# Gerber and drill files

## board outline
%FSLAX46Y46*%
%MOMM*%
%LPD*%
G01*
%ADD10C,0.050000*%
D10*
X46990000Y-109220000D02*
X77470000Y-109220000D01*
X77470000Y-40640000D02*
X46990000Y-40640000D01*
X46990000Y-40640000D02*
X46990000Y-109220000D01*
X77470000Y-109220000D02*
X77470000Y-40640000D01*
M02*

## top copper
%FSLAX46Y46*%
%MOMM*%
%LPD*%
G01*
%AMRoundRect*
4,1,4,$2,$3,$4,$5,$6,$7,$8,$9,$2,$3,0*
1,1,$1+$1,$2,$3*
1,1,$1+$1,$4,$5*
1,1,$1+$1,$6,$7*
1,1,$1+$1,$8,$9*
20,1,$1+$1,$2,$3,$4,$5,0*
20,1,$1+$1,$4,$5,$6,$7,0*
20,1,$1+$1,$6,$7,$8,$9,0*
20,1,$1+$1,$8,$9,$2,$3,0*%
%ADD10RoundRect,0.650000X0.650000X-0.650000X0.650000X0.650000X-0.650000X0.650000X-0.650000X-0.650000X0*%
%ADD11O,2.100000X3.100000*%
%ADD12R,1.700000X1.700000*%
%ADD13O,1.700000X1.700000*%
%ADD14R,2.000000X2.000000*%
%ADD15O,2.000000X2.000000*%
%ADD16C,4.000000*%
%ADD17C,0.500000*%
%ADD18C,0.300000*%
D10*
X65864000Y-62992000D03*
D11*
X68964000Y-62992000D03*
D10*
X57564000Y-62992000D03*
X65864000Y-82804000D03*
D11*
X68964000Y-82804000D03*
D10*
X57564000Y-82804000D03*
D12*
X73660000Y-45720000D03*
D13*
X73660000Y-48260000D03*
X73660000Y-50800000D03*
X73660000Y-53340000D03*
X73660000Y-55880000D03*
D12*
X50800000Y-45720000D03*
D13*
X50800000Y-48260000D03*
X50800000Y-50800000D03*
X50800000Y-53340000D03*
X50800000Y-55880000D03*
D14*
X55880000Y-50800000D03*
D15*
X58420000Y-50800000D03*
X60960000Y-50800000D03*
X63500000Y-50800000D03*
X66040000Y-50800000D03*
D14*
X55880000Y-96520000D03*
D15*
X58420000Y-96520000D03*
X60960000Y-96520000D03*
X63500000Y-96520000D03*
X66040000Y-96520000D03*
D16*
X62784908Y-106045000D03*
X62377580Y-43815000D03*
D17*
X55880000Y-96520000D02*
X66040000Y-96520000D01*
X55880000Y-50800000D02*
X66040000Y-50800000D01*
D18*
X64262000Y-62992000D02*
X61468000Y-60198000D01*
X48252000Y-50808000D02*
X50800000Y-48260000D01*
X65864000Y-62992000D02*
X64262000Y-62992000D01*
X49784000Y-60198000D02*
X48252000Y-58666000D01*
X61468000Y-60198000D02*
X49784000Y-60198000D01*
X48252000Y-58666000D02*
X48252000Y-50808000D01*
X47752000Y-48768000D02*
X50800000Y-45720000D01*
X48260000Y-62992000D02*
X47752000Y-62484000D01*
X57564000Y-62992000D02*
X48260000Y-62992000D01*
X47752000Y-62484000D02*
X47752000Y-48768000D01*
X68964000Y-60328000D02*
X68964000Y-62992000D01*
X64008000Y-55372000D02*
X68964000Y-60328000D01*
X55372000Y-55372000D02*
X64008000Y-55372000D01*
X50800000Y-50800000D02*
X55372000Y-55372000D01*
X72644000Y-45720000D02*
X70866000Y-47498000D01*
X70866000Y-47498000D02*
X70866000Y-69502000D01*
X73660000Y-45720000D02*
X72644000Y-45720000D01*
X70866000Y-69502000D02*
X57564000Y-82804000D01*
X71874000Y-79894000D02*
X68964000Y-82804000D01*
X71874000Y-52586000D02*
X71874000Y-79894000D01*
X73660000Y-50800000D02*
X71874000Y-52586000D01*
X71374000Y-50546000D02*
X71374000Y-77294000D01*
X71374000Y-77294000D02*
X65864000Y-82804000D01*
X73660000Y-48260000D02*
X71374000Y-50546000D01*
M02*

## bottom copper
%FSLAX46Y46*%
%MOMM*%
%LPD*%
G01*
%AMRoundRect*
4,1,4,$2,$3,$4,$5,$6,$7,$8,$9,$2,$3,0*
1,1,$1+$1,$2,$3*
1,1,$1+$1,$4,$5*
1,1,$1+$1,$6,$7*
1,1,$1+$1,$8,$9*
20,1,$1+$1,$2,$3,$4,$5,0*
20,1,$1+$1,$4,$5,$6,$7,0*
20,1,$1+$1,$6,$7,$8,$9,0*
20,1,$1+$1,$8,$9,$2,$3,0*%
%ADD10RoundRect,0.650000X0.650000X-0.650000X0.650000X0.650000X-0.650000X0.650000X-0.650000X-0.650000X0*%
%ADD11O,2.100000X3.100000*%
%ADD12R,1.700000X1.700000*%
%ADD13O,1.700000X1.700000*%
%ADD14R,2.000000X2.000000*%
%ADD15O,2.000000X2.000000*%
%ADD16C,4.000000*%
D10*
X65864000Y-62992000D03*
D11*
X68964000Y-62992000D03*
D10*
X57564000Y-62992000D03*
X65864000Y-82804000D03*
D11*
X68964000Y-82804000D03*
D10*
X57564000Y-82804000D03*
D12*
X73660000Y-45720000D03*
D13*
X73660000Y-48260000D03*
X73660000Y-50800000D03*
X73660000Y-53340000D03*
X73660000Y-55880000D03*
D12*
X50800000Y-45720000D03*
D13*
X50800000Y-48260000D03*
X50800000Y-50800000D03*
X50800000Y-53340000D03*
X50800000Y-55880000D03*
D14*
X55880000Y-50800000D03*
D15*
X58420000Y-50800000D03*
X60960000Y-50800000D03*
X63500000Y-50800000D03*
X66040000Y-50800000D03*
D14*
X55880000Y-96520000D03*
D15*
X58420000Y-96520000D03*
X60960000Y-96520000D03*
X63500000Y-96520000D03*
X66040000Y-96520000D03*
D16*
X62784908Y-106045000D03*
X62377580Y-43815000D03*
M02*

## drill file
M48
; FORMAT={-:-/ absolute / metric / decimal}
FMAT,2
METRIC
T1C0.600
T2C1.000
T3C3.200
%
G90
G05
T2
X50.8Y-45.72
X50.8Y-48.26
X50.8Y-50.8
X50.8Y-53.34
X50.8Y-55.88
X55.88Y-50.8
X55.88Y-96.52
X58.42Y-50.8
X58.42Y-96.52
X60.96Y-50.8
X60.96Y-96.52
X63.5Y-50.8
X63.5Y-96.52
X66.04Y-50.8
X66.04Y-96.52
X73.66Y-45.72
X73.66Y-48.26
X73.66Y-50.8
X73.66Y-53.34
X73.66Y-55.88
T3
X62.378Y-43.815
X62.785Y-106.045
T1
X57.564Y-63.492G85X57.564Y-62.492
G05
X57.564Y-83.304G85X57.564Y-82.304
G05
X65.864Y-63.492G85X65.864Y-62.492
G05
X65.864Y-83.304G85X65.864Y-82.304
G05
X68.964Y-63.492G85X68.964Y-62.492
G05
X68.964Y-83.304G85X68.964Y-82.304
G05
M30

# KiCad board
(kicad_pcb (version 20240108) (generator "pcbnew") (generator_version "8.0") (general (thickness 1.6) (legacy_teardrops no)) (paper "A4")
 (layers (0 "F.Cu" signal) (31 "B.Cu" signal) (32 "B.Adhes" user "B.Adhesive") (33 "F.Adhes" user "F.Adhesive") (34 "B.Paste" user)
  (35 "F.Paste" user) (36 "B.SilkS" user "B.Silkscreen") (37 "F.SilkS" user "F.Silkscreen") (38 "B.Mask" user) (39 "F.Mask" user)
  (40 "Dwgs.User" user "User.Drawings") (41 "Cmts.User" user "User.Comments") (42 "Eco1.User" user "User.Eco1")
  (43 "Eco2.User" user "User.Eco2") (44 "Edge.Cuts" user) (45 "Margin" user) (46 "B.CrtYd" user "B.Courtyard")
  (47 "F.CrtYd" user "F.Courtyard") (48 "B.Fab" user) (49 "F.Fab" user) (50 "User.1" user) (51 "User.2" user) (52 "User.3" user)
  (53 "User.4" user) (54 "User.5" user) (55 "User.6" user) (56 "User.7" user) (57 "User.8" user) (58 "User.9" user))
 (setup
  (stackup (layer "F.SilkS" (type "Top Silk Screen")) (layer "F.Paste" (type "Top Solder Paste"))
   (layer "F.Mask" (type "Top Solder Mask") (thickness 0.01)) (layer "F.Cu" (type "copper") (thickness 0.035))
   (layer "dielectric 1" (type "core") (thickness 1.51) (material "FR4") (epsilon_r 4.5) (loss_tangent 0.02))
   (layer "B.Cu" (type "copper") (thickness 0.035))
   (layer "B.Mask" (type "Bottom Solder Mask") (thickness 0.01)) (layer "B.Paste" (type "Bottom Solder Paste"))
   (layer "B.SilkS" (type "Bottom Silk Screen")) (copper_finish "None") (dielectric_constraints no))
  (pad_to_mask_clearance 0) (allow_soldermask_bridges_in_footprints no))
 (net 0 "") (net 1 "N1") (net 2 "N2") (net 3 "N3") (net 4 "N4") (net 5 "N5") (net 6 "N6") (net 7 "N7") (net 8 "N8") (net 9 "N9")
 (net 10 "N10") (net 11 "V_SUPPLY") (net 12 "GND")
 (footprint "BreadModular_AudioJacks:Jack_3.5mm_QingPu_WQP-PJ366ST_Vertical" (layer "F.Cu") (at 62.484 62.992 90)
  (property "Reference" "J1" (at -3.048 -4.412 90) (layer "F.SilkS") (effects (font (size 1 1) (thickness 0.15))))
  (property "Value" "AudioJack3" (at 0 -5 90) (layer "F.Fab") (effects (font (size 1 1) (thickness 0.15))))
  (pad "R" thru_hole roundrect (at 0 3.38 90) (size 2.6 2.6) (drill oval 1.6 0.6) (layers "*.Cu" "*.Mask") (remove_unused_layers no)
   (roundrect_rratio 0.25) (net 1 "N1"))
  (pad "S" thru_hole oval (at 0 6.48 90) (size 3.1 2.1) (drill oval 1.6 0.6) (layers "*.Cu" "*.Mask") (remove_unused_layers no) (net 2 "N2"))
  (pad "T" thru_hole roundrect (at 0 -4.92 90) (size 2.6 2.6) (drill oval 1.6 0.6) (layers "*.Cu" "*.Mask") (remove_unused_layers no)
   (roundrect_rratio 0.25) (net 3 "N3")))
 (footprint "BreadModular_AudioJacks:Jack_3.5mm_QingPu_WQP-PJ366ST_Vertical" (layer "F.Cu") (at 62.484 82.804 90)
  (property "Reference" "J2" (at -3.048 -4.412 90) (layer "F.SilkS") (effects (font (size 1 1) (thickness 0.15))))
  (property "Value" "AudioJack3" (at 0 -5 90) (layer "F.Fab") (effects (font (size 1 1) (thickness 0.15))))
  (pad "R" thru_hole roundrect (at 0 3.38 90) (size 2.6 2.6) (drill oval 1.6 0.6) (layers "*.Cu" "*.Mask") (remove_unused_layers no)
   (roundrect_rratio 0.25) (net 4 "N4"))
  (pad "S" thru_hole oval (at 0 6.48 90) (size 3.1 2.1) (drill oval 1.6 0.6) (layers "*.Cu" "*.Mask") (remove_unused_layers no) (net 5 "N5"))
  (pad "T" thru_hole roundrect (at 0 -4.92 90) (size 2.6 2.6) (drill oval 1.6 0.6) (layers "*.Cu" "*.Mask") (remove_unused_layers no)
   (roundrect_rratio 0.25) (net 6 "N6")))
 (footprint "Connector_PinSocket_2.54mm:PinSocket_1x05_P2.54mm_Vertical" (layer "F.Cu") (at 73.66 45.72)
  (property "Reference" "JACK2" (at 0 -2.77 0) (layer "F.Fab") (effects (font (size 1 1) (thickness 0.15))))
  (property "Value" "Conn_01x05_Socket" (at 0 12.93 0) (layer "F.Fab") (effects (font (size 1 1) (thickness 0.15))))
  (pad "1" thru_hole rect (at 0 0) (size 1.7 1.7) (drill 1) (layers "*.Cu" "*.Mask") (remove_unused_layers no) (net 6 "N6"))
  (pad "2" thru_hole oval (at 0 2.54) (size 1.7 1.7) (drill 1) (layers "*.Cu" "*.Mask") (remove_unused_layers no) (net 4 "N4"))
  (pad "3" thru_hole oval (at 0 5.08) (size 1.7 1.7) (drill 1) (layers "*.Cu" "*.Mask") (remove_unused_layers no) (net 5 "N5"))
  (pad "4" thru_hole oval (at 0 7.62) (size 1.7 1.7) (drill 1) (layers "*.Cu" "*.Mask") (remove_unused_layers no) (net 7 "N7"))
  (pad "5" thru_hole oval (at 0 10.16) (size 1.7 1.7) (drill 1) (layers "*.Cu" "*.Mask") (remove_unused_layers no) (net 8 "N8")))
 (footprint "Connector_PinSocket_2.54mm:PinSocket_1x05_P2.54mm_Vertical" (layer "F.Cu") (at 50.8 45.72)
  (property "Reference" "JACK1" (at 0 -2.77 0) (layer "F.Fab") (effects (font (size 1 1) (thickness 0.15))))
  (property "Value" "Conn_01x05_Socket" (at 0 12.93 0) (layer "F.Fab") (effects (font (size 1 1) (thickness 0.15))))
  (pad "1" thru_hole rect (at 0 0) (size 1.7 1.7) (drill 1) (layers "*.Cu" "*.Mask") (remove_unused_layers no) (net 3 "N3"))
  (pad "2" thru_hole oval (at 0 2.54) (size 1.7 1.7) (drill 1) (layers "*.Cu" "*.Mask") (remove_unused_layers no) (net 1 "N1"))
  (pad "3" thru_hole oval (at 0 5.08) (size 1.7 1.7) (drill 1) (layers "*.Cu" "*.Mask") (remove_unused_layers no) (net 2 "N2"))
  (pad "4" thru_hole oval (at 0 7.62) (size 1.7 1.7) (drill 1) (layers "*.Cu" "*.Mask") (remove_unused_layers no) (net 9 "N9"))
  (pad "5" thru_hole oval (at 0 10.16) (size 1.7 1.7) (drill 1) (layers "*.Cu" "*.Mask") (remove_unused_layers no) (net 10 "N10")))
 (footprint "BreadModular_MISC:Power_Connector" (layer "B.Cu") (at 55.88 50.8 -90)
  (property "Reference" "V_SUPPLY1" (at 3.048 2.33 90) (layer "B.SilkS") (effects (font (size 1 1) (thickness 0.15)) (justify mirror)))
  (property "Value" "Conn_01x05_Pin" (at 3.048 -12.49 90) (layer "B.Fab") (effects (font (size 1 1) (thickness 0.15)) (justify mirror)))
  (pad "1" thru_hole rect (at 0 0 270) (size 2 2) (drill 1) (layers "*.Cu" "*.Mask") (remove_unused_layers no) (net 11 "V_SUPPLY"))
  (pad "2" thru_hole oval (at 0 -2.54 270) (size 2 2) (drill 1) (layers "*.Cu" "*.Mask") (remove_unused_layers no) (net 11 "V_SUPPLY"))
  (pad "3" thru_hole oval (at 0 -5.08 270) (size 2 2) (drill 1) (layers "*.Cu" "*.Mask") (remove_unused_layers no) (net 11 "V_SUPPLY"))
  (pad "4" thru_hole oval (at 0 -7.62 270) (size 2 2) (drill 1) (layers "*.Cu" "*.Mask") (remove_unused_layers no) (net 11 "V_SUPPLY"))
  (pad "5" thru_hole oval (at 0 -10.16 270) (size 2 2) (drill 1) (layers "*.Cu" "*.Mask") (remove_unused_layers no) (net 11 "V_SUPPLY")))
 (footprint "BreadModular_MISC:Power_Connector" (layer "B.Cu") (at 55.88 96.52 -90)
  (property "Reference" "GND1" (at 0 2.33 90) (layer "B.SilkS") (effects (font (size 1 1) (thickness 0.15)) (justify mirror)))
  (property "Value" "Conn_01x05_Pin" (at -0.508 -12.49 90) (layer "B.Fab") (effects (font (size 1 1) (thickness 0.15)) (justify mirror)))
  (pad "1" thru_hole rect (at 0 0 270) (size 2 2) (drill 1) (layers "*.Cu" "*.Mask") (remove_unused_layers no) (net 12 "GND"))
  (pad "2" thru_hole oval (at 0 -2.54 270) (size 2 2) (drill 1) (layers "*.Cu" "*.Mask") (remove_unused_layers no) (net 12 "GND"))
  (pad "3" thru_hole oval (at 0 -5.08 270) (size 2 2) (drill 1) (layers "*.Cu" "*.Mask") (remove_unused_layers no) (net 12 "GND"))
  (pad "4" thru_hole oval (at 0 -7.62 270) (size 2 2) (drill 1) (layers "*.Cu" "*.Mask") (remove_unused_layers no) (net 12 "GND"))
  (pad "5" thru_hole oval (at 0 -10.16 270) (size 2 2) (drill 1) (layers "*.Cu" "*.Mask") (remove_unused_layers no) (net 12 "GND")))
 (gr_line (start 46.99 109.22) (end 77.47 109.22) (stroke (width 0.05) (type default)) (layer "Edge.Cuts"))
 (gr_line (start 77.47 40.64) (end 46.99 40.64) (stroke (width 0.05) (type default)) (layer "Edge.Cuts"))
 (gr_line (start 46.99 40.64) (end 46.99 109.22) (stroke (width 0.05) (type default)) (layer "Edge.Cuts"))
 (gr_line (start 77.47 109.22) (end 77.47 40.64) (stroke (width 0.05) (type default)) (layer "Edge.Cuts"))
 (via (at 62.784908 106.045) (size 4) (drill 3.2) (layers "F.Cu" "B.Cu") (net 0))
 (via (at 62.37758 43.815) (size 4) (drill 3.2) (layers "F.Cu" "B.Cu") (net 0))
 (segment (start 55.88 96.52) (end 66.04 96.52) (width 0.5) (layer "F.Cu") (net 12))
 (segment (start 55.88 50.8) (end 66.04 50.8) (width 0.5) (layer "F.Cu") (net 11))
 (segment (start 64.262 62.992) (end 61.468 60.198) (width 0.3) (layer "F.Cu") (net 1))
 (segment (start 48.252 50.808) (end 50.8 48.26) (width 0.3) (layer "F.Cu") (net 1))
 (segment (start 65.864 62.992) (end 64.262 62.992) (width 0.3) (layer "F.Cu") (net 1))
 (segment (start 49.784 60.198) (end 48.252 58.666) (width 0.3) (layer "F.Cu") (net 1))
 (segment (start 61.468 60.198) (end 49.784 60.198) (width 0.3) (layer "F.Cu") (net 1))
 (segment (start 48.252 58.666) (end 48.252 50.808) (width 0.3) (layer "F.Cu") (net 1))
 (segment (start 47.752 48.768) (end 50.8 45.72) (width 0.3) (layer "F.Cu") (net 3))
 (segment (start 48.26 62.992) (end 47.752 62.484) (width 0.3) (layer "F.Cu") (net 3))
 (segment (start 57.564 62.992) (end 48.26 62.992) (width 0.3) (layer "F.Cu") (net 3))
 (segment (start 47.752 62.484) (end 47.752 48.768) (width 0.3) (layer "F.Cu") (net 3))
 (segment (start 68.964 60.328) (end 68.964 62.992) (width 0.3) (layer "F.Cu") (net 2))
 (segment (start 64.008 55.372) (end 68.964 60.328) (width 0.3) (layer "F.Cu") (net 2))
 (segment (start 55.372 55.372) (end 64.008 55.372) (width 0.3) (layer "F.Cu") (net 2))
 (segment (start 50.8 50.8) (end 55.372 55.372) (width 0.3) (layer "F.Cu") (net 2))
 (segment (start 72.644 45.72) (end 70.866 47.498) (width 0.3) (layer "F.Cu") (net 6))
 (segment (start 70.866 47.498) (end 70.866 69.502) (width 0.3) (layer "F.Cu") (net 6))
 (segment (start 73.66 45.72) (end 72.644 45.72) (width 0.3) (layer "F.Cu") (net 6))
 (segment (start 70.866 69.502) (end 57.564 82.804) (width 0.3) (layer "F.Cu") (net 6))
 (segment (start 71.874 79.894) (end 68.964 82.804) (width 0.3) (layer "F.Cu") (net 5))
 (segment (start 71.874 52.586) (end 71.874 79.894) (width 0.3) (layer "F.Cu") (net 5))
 (segment (start 73.66 50.8) (end 71.874 52.586) (width 0.3) (layer "F.Cu") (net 5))
 (segment (start 71.374 50.546) (end 71.374 77.294) (width 0.3) (layer "F.Cu") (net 4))
 (segment (start 71.374 77.294) (end 65.864 82.804) (width 0.3) (layer "F.Cu") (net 4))
 (segment (start 73.66 48.26) (end 71.374 50.546) (width 0.3) (layer "F.Cu") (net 4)))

